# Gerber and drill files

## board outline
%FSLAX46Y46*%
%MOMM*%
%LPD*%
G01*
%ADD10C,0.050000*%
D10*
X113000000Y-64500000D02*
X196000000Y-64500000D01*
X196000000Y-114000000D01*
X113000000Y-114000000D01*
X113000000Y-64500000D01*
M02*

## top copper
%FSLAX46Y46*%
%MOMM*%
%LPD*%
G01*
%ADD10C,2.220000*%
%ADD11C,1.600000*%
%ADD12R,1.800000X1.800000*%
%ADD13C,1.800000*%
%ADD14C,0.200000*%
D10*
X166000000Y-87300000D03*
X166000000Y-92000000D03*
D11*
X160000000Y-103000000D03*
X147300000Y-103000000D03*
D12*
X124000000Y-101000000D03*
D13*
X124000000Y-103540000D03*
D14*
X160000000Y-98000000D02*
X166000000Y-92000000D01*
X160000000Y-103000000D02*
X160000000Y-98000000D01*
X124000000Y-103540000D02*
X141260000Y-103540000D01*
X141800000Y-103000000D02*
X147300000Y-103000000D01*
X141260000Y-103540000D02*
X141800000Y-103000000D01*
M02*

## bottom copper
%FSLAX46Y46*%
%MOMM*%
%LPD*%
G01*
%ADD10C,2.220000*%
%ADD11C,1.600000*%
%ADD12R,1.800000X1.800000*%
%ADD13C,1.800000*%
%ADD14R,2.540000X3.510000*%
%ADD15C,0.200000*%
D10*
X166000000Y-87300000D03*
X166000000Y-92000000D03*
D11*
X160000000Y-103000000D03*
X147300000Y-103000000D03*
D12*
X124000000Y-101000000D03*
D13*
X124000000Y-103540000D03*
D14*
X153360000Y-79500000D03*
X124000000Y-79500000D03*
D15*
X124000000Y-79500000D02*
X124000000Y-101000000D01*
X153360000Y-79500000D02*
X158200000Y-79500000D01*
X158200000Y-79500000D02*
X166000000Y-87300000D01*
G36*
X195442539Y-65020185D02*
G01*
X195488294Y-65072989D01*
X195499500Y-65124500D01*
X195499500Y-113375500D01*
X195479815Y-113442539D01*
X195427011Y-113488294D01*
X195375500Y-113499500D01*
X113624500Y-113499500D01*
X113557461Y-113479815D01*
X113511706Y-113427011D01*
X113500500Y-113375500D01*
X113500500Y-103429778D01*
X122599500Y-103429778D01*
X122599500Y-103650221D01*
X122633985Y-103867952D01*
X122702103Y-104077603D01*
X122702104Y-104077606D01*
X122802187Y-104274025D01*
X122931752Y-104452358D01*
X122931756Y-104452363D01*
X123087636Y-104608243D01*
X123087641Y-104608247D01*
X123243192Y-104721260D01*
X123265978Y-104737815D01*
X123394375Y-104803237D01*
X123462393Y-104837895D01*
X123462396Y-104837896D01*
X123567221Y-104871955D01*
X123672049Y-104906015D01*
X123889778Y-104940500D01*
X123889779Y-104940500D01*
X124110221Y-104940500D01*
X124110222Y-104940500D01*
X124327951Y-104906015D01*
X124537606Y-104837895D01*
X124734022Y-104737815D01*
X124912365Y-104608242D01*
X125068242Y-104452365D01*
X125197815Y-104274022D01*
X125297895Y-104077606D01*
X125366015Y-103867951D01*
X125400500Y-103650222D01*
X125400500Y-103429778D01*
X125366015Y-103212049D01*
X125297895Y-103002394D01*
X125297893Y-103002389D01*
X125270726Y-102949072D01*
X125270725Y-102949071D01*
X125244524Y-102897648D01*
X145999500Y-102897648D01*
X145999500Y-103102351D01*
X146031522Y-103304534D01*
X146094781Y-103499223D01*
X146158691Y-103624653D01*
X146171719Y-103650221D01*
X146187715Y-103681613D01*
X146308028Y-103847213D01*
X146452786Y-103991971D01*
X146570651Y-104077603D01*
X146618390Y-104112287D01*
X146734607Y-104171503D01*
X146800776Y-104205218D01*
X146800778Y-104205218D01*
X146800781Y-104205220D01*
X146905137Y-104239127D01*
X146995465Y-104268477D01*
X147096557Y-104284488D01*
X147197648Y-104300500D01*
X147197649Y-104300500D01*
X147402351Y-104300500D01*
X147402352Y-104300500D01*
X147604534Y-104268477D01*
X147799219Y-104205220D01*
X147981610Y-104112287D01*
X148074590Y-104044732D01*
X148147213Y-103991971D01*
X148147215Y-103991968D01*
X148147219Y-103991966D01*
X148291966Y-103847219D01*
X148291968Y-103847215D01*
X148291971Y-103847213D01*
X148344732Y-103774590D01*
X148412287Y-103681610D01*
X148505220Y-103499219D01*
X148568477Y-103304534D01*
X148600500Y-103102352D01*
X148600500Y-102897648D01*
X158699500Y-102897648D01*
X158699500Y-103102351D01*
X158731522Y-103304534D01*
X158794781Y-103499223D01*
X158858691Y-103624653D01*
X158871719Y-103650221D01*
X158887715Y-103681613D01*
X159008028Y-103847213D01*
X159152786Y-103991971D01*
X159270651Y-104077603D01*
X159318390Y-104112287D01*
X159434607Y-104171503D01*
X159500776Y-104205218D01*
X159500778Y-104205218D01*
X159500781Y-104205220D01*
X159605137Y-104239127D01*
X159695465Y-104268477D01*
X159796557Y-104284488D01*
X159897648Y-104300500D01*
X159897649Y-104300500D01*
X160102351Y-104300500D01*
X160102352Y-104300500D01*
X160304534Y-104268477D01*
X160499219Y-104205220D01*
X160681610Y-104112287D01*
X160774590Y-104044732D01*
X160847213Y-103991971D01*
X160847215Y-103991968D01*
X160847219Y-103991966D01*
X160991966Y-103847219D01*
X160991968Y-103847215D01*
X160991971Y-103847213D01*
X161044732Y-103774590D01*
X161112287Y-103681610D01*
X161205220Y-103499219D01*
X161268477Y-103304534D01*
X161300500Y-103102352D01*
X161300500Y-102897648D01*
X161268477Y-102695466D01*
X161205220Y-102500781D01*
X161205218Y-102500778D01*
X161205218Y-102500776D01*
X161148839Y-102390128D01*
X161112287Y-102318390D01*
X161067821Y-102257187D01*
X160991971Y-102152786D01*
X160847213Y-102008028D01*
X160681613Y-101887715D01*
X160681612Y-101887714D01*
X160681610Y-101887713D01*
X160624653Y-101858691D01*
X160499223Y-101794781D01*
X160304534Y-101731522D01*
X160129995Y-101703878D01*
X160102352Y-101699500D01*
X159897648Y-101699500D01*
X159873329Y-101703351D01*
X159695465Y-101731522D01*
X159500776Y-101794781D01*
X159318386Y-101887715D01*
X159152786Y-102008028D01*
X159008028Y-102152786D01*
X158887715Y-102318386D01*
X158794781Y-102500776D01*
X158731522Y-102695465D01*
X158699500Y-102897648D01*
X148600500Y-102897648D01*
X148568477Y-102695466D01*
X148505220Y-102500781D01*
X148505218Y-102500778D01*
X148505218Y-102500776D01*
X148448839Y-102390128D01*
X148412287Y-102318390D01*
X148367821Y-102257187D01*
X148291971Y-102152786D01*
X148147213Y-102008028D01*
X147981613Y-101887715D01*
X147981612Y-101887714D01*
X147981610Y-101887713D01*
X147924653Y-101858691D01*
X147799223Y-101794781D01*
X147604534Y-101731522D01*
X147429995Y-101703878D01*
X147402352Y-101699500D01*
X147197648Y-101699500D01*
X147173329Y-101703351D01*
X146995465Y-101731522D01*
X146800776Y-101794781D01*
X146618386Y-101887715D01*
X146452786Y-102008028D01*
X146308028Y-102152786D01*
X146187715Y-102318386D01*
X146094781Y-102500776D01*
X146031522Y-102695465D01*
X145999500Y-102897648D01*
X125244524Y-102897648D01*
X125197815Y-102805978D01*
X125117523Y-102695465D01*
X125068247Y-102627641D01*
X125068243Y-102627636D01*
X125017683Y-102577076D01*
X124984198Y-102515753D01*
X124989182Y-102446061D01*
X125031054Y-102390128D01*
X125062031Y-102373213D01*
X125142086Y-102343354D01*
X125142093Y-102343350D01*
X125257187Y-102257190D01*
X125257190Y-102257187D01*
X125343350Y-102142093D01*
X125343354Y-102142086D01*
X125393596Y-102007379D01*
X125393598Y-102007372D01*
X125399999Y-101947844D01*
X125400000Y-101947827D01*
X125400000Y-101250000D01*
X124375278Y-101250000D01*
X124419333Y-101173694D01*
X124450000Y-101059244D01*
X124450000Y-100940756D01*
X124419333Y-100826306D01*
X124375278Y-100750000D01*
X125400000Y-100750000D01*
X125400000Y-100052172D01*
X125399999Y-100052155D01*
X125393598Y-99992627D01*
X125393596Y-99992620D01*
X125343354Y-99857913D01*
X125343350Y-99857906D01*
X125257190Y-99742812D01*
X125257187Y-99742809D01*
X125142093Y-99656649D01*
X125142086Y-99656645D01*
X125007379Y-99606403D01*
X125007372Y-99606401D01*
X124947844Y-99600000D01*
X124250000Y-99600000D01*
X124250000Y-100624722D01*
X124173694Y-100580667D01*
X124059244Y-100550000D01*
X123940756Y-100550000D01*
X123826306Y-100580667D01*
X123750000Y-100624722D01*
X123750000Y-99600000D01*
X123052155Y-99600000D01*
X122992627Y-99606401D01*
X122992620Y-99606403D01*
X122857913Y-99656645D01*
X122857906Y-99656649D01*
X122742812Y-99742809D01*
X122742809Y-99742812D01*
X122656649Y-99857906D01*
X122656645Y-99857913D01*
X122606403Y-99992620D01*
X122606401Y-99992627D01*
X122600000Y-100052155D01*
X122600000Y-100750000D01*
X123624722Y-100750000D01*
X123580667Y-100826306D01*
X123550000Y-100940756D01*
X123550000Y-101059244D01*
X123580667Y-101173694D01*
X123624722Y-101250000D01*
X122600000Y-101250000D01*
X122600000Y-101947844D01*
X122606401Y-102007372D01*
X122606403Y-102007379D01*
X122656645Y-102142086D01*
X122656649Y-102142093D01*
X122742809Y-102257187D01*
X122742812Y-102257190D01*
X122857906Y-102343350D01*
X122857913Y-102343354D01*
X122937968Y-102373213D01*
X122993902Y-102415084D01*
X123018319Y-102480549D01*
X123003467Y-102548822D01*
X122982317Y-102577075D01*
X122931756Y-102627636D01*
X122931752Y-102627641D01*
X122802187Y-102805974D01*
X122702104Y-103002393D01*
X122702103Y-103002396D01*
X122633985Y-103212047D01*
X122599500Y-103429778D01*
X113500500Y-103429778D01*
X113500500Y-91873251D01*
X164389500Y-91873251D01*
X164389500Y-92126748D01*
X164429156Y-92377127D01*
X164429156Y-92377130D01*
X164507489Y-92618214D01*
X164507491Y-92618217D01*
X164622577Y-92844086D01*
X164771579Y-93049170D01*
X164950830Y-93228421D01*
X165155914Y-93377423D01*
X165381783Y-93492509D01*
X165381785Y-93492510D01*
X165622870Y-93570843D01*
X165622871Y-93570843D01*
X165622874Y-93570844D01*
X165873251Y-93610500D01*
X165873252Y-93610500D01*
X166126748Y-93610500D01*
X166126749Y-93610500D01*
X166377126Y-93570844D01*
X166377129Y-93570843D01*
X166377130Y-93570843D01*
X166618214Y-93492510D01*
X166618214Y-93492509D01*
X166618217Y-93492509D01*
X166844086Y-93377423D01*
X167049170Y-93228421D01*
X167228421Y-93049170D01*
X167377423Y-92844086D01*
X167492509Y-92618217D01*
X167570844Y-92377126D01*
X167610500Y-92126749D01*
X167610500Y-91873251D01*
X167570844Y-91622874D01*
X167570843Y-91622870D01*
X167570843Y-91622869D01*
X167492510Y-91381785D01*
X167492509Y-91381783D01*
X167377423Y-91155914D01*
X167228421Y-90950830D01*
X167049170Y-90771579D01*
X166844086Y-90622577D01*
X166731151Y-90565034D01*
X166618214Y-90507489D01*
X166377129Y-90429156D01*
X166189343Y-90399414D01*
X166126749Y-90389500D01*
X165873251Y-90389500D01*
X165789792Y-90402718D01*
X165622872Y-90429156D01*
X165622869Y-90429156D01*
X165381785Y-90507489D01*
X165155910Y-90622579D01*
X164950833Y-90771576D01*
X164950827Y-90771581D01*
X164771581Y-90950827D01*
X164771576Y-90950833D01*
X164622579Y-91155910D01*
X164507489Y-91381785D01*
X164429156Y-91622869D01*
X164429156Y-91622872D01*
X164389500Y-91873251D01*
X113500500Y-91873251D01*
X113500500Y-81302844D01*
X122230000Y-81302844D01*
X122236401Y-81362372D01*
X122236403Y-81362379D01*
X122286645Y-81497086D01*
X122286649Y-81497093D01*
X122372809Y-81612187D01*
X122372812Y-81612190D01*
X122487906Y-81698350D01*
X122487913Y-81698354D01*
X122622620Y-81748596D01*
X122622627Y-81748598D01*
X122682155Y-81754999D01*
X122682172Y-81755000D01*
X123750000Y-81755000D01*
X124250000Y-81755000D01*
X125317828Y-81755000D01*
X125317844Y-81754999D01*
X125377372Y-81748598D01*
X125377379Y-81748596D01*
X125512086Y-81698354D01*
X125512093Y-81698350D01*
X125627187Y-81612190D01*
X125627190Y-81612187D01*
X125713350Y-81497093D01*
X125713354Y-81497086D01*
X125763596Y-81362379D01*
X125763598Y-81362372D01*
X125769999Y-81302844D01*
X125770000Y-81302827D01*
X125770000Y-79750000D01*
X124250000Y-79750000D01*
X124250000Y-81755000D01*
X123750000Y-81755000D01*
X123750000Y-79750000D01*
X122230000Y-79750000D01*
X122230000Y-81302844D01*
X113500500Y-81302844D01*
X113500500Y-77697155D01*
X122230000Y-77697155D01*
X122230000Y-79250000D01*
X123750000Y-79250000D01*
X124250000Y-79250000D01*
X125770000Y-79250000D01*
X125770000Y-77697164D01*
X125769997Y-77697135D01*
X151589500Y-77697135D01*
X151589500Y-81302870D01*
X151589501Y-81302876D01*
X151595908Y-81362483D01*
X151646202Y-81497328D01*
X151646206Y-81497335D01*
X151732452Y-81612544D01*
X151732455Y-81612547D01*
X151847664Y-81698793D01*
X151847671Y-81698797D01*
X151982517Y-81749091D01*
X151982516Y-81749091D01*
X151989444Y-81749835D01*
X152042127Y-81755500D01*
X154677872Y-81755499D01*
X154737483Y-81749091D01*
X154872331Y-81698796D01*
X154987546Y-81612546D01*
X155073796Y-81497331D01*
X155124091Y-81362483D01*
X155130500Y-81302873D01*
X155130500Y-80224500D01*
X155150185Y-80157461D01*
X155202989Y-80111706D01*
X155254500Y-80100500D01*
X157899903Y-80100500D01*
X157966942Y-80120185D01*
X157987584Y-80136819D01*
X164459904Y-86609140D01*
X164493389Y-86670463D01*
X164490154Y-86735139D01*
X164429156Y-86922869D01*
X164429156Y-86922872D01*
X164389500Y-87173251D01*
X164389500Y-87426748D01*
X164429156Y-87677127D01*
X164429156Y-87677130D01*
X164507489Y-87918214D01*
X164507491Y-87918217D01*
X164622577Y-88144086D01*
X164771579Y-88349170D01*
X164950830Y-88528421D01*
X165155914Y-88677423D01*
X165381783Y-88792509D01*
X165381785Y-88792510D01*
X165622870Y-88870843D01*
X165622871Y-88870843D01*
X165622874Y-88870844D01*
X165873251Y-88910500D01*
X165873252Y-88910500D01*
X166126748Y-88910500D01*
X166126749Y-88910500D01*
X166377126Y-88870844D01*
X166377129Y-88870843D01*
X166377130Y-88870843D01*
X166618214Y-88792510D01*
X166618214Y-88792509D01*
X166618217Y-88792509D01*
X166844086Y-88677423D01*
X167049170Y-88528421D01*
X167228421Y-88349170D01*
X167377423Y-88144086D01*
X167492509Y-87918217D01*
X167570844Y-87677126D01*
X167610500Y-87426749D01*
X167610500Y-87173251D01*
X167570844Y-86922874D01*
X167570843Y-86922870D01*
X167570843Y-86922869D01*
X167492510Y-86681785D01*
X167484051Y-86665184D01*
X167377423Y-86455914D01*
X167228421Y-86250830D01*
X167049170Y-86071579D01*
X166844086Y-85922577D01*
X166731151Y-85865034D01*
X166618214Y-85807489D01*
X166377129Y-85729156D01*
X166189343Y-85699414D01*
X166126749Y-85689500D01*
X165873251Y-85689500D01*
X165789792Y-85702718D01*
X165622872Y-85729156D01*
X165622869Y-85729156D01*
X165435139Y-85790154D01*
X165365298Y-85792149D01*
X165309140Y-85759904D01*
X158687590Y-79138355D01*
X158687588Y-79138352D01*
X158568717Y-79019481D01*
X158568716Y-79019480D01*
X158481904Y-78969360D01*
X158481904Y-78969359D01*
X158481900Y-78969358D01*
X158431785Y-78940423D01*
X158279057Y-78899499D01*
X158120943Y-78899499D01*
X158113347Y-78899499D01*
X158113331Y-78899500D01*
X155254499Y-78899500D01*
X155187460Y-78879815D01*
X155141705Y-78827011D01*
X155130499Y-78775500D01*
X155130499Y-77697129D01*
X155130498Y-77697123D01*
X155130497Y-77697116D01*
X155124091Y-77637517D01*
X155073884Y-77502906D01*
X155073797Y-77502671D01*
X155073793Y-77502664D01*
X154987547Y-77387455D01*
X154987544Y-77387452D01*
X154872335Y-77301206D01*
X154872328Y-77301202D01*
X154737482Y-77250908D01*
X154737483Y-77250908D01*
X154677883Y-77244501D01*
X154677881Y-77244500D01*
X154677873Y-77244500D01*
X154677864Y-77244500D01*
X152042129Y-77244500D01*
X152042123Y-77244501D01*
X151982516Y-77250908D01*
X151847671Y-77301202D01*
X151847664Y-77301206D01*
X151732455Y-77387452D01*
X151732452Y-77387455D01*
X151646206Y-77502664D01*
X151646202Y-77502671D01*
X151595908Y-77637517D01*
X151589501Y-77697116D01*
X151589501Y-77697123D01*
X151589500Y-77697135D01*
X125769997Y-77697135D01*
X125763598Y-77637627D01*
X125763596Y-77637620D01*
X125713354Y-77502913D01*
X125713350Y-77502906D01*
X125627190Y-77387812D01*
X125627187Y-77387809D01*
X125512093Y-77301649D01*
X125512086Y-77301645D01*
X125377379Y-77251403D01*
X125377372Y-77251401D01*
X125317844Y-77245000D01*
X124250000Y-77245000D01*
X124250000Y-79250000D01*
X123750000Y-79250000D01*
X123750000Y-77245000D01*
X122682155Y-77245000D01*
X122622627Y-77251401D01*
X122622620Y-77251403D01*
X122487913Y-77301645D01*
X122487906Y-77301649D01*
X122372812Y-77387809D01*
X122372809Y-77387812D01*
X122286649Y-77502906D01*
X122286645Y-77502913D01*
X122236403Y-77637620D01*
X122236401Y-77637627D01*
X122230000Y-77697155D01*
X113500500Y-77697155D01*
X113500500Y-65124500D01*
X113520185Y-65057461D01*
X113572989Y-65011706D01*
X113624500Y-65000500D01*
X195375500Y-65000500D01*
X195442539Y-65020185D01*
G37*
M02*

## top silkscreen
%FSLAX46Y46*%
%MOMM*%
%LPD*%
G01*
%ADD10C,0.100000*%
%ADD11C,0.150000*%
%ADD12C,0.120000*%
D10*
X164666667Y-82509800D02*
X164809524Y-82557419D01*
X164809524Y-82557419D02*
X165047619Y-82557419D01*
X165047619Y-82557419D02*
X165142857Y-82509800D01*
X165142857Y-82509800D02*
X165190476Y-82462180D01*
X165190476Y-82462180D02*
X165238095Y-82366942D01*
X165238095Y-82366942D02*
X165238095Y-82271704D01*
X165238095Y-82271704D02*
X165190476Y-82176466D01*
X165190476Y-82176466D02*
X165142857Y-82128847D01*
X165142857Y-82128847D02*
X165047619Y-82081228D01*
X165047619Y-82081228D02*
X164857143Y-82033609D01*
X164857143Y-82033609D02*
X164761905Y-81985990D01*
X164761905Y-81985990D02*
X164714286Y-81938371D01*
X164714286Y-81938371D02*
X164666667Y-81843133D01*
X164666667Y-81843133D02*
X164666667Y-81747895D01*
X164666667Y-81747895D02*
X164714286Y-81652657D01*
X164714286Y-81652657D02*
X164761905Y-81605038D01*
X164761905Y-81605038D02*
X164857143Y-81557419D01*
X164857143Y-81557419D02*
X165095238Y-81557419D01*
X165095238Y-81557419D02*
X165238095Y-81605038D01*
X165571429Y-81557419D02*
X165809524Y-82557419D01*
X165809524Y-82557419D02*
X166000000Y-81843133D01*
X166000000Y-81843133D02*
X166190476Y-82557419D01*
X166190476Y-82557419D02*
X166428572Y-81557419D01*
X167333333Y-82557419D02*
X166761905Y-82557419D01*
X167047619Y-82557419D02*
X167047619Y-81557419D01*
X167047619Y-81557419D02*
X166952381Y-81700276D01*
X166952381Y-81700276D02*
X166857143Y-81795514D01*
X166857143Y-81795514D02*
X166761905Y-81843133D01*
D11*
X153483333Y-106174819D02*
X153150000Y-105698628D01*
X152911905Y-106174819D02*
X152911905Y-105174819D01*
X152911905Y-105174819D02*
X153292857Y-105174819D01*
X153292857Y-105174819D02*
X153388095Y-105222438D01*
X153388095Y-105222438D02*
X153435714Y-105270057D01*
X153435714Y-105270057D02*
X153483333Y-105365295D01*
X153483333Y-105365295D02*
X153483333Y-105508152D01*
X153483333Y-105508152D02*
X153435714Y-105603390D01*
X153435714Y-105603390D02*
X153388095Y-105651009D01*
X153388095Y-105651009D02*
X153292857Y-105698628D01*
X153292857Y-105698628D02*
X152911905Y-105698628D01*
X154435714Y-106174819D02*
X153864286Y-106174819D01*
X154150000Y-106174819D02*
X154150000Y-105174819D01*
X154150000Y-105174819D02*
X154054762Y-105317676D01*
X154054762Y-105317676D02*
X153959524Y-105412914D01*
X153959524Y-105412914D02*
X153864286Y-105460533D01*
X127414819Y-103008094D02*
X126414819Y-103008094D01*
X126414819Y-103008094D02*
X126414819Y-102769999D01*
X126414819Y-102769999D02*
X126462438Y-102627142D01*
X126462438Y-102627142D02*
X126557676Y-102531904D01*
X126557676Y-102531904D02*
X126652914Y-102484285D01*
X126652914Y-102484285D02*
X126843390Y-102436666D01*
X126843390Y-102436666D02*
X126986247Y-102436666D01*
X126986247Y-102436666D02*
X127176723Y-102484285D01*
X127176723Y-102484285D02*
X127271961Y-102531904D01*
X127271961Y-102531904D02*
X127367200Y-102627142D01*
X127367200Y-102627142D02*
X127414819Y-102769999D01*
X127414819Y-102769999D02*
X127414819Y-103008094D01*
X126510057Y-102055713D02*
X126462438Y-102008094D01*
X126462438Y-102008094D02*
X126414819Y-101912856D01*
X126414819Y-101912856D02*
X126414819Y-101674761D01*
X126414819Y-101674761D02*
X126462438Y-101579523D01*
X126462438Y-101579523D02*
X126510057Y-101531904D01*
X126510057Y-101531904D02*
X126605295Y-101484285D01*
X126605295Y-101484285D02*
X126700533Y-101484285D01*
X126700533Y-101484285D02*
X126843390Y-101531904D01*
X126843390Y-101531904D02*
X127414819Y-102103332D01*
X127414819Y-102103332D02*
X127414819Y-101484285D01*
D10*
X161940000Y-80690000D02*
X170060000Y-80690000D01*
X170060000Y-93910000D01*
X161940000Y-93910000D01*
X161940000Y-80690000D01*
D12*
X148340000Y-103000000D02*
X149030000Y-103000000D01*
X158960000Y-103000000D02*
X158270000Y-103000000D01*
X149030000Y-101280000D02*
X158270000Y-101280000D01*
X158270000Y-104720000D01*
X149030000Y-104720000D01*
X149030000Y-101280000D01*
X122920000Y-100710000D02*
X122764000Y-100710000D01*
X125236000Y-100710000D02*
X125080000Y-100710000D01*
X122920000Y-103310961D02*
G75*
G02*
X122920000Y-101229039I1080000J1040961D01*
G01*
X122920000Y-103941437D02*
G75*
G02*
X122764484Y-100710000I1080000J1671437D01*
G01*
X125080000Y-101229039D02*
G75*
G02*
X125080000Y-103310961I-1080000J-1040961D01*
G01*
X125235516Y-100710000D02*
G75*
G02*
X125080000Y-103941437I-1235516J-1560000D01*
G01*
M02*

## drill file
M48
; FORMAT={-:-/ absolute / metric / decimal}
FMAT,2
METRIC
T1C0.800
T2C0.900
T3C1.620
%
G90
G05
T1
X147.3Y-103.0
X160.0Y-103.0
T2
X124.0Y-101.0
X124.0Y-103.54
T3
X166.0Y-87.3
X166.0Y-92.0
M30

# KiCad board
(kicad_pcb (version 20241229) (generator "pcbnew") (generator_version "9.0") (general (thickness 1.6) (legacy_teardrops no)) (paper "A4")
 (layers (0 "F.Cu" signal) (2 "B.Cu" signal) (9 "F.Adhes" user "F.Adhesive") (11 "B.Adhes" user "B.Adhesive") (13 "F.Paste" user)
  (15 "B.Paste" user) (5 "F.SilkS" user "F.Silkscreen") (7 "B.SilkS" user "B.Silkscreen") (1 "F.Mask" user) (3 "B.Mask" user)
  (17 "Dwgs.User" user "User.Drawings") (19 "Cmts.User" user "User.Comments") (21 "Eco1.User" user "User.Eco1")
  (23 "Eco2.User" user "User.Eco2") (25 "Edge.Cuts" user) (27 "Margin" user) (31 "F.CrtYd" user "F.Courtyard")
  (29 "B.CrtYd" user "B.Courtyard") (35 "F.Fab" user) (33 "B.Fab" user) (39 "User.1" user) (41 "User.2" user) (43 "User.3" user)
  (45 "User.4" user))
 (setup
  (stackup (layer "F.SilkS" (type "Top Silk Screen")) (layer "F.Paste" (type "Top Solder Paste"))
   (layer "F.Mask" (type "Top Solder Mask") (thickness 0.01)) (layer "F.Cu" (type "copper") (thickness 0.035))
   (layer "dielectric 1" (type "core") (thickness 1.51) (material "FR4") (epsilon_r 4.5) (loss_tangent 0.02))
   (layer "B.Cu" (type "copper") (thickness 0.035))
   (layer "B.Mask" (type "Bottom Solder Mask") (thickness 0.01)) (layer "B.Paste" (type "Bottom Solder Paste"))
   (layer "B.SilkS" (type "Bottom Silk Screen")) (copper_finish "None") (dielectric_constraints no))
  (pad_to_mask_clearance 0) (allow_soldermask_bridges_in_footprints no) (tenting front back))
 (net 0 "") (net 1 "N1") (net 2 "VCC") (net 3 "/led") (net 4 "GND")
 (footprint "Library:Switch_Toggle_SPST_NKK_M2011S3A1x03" (layer "F.Cu") (at 166 82.6)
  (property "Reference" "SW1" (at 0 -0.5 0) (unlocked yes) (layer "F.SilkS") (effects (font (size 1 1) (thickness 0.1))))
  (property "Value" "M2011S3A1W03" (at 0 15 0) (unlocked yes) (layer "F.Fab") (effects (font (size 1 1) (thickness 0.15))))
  (fp_rect (start -4.06 -1.91) (end 4.06 11.31) (stroke (width 0.1) (type default)) (fill no) (layer "F.SilkS"))
  (pad "2" thru_hole circle (at 0 4.7) (size 2.22 2.22) (drill 1.62) (layers "*.Cu" "*.Mask") (remove_unused_layers no) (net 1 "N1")
   (thermal_bridge_angle 90))
  (pad "3" thru_hole circle (at 0 9.4) (size 2.22 2.22) (drill 1.62) (layers "*.Cu" "*.Mask") (remove_unused_layers no) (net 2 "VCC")))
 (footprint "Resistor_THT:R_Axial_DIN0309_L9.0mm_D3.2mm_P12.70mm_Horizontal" (layer "F.Cu") (at 160 103 180)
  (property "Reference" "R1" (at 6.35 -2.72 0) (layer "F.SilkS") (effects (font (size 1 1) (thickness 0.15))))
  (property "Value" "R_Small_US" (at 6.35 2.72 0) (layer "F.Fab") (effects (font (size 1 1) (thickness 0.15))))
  (fp_line (start 11.66 0) (end 10.97 0) (stroke (width 0.12) (type solid)) (layer "F.SilkS"))
  (fp_line (start 1.04 0) (end 1.73 0) (stroke (width 0.12) (type solid)) (layer "F.SilkS"))
  (fp_rect (start 1.73 -1.72) (end 10.97 1.72) (stroke (width 0.12) (type solid)) (fill no) (layer "F.SilkS"))
  (pad "1" thru_hole circle (at 0 0 180) (size 1.6 1.6) (drill 0.8) (layers "*.Cu" "*.Mask") (remove_unused_layers no) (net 2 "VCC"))
  (pad "2" thru_hole circle (at 12.7 0 180) (size 1.6 1.6) (drill 0.8) (layers "*.Cu" "*.Mask") (remove_unused_layers no) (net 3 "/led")))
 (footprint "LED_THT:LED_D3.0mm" (layer "F.Cu") (at 124 101 -90)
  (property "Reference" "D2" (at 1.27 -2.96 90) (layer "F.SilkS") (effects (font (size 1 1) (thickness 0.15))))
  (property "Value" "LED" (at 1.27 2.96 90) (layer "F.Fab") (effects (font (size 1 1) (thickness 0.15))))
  (fp_line (start -0.29 1.08) (end -0.29 1.236) (stroke (width 0.12) (type solid)) (layer "F.SilkS"))
  (fp_line (start -0.29 -1.236) (end -0.29 -1.08) (stroke (width 0.12) (type solid)) (layer "F.SilkS"))
  (fp_arc (start 2.310961 1.08) (mid 1.27 1.5) (end 0.229039 1.08) (stroke (width 0.12) (type solid)) (layer "F.SilkS"))
  (fp_arc (start 2.941437 1.08) (mid 1.36566 1.987699) (end -0.29 1.235516) (stroke (width 0.12) (type solid)) (layer "F.SilkS"))
  (fp_arc (start 0.229039 -1.08) (mid 1.27 -1.5) (end 2.310961 -1.08) (stroke (width 0.12) (type solid)) (layer "F.SilkS"))
  (fp_arc (start -0.29 -1.235516) (mid 1.36566 -1.987699) (end 2.941437 -1.08) (stroke (width 0.12) (type solid)) (layer "F.SilkS"))
  (pad "1" thru_hole rect (at 0 0 270) (size 1.8 1.8) (drill 0.9) (layers "*.Cu" "*.Mask") (remove_unused_layers no) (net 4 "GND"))
  (pad "2" thru_hole circle (at 2.54 0 270) (size 1.8 1.8) (drill 0.9) (layers "*.Cu" "*.Mask") (remove_unused_layers no) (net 3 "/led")))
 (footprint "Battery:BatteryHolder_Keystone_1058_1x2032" (layer "B.Cu") (at 138.68 79.5 180)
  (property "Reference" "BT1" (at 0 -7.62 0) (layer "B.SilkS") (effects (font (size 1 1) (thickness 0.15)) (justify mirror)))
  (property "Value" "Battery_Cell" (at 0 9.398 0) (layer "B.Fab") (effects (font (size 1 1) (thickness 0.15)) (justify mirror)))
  (pad "1" smd rect (at -14.68 0 180) (size 2.54 3.51) (layers "B.Cu" "B.Mask" "B.Paste") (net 1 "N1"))
  (pad "2" smd rect (at 14.68 0 180) (size 2.54 3.51) (layers "B.Cu" "B.Mask" "B.Paste") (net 4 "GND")))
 (gr_rect (start 113 64.5) (end 196 114) (stroke (width 0.05) (type default)) (fill no) (layer "Edge.Cuts"))
 (segment (start 160 98) (end 166 92) (width 0.2) (layer "F.Cu") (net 2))
 (segment (start 160 103) (end 160 98) (width 0.2) (layer "F.Cu") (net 2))
 (segment (start 124 79.5) (end 124 101) (width 0.2) (layer "B.Cu") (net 4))
 (segment (start 124 103.54) (end 141.26 103.54) (width 0.2) (layer "F.Cu") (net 3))
 (segment (start 141.8 103) (end 147.3 103) (width 0.2) (layer "F.Cu") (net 3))
 (segment (start 141.26 103.54) (end 141.8 103) (width 0.2) (layer "F.Cu") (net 3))
 (segment (start 153.36 79.5) (end 158.2 79.5) (width 0.2) (layer "B.Cu") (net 1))
 (segment (start 158.2 79.5) (end 166 87.3) (width 0.2) (layer "B.Cu") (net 1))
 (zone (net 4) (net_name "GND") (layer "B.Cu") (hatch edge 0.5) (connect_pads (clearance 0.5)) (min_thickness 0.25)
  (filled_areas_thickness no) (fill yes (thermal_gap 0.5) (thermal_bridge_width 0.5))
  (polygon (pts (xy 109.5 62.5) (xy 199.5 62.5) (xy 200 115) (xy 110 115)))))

